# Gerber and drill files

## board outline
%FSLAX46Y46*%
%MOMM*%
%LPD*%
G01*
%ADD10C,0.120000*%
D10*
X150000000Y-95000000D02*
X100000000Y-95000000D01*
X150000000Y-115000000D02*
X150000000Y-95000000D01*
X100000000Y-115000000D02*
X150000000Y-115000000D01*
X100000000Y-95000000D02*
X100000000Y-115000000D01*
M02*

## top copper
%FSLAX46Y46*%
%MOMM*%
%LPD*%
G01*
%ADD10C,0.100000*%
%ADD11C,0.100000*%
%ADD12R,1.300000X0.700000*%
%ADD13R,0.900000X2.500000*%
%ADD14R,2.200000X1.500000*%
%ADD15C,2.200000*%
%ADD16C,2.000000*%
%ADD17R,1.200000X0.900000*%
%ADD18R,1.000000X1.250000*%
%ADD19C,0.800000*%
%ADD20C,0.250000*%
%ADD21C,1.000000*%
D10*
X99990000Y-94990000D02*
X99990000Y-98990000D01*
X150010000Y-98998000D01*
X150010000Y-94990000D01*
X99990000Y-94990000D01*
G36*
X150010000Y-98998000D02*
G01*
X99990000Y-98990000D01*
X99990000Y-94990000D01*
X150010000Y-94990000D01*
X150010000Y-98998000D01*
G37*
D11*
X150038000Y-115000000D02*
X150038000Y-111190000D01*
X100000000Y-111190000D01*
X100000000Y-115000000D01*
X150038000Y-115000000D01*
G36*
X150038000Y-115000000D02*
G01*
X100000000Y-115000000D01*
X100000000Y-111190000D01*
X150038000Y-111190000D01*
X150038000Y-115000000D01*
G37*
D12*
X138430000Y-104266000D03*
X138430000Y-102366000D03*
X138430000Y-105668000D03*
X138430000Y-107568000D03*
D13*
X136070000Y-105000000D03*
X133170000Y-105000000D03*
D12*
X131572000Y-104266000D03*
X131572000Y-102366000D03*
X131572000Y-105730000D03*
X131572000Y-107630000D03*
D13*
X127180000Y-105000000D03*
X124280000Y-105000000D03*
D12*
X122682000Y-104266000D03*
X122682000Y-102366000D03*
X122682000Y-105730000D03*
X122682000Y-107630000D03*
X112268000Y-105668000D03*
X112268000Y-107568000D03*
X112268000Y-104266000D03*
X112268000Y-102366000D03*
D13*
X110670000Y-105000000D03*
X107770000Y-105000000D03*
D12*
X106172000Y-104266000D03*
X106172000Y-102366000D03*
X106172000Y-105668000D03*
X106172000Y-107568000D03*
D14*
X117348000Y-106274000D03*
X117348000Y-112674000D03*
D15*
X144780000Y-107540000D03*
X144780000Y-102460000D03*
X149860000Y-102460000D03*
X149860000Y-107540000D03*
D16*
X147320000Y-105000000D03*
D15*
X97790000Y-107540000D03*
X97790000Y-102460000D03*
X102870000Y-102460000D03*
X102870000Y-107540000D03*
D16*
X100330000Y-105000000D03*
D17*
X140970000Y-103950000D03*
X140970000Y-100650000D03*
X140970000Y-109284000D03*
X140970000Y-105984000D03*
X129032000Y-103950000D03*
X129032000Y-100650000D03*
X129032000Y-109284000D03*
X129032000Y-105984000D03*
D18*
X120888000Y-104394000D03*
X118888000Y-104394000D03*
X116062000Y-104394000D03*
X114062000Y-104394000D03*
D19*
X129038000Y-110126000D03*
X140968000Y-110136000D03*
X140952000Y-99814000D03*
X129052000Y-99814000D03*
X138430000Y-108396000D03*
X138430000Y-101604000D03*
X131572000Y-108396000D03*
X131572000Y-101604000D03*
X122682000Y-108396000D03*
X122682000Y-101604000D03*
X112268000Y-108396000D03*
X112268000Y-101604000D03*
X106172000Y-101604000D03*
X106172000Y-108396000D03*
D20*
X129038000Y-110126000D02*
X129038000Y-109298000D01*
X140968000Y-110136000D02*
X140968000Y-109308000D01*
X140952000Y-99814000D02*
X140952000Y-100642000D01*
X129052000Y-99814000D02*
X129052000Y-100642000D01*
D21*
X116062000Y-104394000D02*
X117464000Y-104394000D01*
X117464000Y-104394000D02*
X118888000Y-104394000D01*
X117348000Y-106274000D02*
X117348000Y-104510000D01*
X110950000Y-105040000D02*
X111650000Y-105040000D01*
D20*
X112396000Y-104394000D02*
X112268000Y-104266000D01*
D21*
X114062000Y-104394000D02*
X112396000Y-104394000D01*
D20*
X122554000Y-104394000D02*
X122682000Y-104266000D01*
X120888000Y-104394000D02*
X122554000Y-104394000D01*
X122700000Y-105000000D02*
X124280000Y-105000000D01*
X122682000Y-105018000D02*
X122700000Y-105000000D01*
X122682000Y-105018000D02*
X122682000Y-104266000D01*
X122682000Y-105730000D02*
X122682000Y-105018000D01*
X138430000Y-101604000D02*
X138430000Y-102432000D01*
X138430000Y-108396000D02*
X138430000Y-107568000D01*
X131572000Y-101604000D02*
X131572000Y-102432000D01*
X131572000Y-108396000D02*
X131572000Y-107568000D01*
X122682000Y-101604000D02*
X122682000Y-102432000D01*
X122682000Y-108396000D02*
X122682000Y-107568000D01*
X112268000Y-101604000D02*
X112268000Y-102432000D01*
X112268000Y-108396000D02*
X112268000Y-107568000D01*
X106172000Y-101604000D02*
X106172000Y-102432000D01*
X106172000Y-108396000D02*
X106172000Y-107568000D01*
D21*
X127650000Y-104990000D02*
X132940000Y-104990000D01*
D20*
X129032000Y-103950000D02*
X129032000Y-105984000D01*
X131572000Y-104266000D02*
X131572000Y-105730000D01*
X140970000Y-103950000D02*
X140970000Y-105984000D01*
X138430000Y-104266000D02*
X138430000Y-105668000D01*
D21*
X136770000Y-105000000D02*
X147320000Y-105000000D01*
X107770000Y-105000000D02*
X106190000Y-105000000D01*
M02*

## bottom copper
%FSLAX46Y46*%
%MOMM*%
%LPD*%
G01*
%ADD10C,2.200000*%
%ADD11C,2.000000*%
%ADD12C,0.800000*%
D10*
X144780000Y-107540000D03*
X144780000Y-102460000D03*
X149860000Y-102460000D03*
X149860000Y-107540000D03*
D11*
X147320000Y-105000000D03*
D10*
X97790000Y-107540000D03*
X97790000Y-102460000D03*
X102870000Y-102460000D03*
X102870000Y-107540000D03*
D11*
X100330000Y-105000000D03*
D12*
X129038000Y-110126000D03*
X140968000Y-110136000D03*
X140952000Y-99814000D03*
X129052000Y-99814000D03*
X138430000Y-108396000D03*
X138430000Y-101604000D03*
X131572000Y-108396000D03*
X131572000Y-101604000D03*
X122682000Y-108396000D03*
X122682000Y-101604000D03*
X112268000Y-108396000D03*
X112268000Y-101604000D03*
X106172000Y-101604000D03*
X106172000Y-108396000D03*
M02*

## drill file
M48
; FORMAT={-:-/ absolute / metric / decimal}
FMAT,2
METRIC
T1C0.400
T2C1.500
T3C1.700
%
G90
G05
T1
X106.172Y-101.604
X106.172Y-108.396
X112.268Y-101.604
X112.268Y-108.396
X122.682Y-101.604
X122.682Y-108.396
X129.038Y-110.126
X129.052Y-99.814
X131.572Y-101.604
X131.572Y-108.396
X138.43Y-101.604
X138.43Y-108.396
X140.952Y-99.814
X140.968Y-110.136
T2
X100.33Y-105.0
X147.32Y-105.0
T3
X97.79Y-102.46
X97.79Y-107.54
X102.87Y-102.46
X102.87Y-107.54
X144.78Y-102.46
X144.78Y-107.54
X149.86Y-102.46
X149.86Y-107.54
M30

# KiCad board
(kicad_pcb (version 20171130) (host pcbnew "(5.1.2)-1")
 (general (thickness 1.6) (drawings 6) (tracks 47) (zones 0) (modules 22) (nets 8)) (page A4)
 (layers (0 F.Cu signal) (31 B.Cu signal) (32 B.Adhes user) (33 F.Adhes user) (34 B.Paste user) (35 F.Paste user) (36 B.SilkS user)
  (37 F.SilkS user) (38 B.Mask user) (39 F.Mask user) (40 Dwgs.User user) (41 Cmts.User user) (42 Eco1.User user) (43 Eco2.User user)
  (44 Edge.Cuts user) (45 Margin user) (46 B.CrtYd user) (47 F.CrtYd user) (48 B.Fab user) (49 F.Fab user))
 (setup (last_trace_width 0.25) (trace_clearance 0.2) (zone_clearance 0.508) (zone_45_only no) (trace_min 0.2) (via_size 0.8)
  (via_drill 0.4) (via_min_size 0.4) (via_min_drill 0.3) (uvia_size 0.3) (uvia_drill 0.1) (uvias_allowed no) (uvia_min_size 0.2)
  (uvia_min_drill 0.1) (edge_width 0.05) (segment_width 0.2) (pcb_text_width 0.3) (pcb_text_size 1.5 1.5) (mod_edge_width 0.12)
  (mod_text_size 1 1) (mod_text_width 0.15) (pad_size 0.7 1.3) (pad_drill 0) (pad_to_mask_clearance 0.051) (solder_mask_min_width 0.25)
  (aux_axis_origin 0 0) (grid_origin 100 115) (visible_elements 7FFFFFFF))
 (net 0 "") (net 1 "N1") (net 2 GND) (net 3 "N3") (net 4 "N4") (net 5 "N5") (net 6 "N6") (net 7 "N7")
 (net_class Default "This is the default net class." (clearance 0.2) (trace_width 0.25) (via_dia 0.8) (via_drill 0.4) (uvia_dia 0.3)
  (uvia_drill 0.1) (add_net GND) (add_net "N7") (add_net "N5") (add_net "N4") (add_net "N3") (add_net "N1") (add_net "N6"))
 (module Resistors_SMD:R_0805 (layer F.Cu) (at 138.43 103.316 90)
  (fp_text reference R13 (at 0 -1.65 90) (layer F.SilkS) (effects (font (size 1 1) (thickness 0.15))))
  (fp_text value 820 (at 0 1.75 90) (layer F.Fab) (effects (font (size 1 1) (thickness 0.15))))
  (pad 1 smd rect (at -0.95 0 90) (size 0.7 1.3) (layers F.Cu F.Paste F.Mask) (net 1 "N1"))
  (pad 2 smd rect (at 0.95 0 90) (size 0.7 1.3) (layers F.Cu F.Paste F.Mask) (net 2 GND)))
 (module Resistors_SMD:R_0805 (layer F.Cu) (at 138.43 106.618 270)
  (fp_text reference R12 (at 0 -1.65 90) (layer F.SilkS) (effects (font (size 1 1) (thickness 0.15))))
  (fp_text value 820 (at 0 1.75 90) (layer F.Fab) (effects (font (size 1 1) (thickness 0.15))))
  (pad 1 smd rect (at -0.95 0 270) (size 0.7 1.3) (layers F.Cu F.Paste F.Mask) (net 1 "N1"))
  (pad 2 smd rect (at 0.95 0 270) (size 0.7 1.3) (layers F.Cu F.Paste F.Mask) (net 2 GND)))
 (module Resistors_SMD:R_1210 (layer F.Cu) (at 134.62 105 180)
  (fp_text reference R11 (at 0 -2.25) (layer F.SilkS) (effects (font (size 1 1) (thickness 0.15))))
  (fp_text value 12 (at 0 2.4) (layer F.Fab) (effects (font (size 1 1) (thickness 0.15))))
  (pad 1 smd rect (at -1.45 0 180) (size 0.9 2.5) (layers F.Cu F.Paste F.Mask) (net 1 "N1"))
  (pad 2 smd rect (at 1.45 0 180) (size 0.9 2.5) (layers F.Cu F.Paste F.Mask) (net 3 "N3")))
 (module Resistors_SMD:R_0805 (layer F.Cu) (at 131.572 103.316 90)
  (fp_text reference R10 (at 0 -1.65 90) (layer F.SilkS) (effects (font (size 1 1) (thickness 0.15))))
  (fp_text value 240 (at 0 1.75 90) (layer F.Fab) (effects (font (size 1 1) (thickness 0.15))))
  (pad 1 smd rect (at -0.95 0 90) (size 0.7 1.3) (layers F.Cu F.Paste F.Mask) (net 3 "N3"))
  (pad 2 smd rect (at 0.95 0 90) (size 0.7 1.3) (layers F.Cu F.Paste F.Mask) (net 2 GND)))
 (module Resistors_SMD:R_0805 (layer F.Cu) (at 131.572 106.68 270)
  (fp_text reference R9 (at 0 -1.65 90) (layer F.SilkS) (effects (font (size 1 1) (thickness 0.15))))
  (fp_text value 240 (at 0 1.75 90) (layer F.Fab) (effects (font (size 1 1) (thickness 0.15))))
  (pad 1 smd rect (at -0.95 0 270) (size 0.7 1.3) (layers F.Cu F.Paste F.Mask) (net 3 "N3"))
  (pad 2 smd rect (at 0.95 0 270) (size 0.7 1.3) (layers F.Cu F.Paste F.Mask) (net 2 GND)))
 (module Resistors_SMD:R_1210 (layer F.Cu) (at 125.73 105 180)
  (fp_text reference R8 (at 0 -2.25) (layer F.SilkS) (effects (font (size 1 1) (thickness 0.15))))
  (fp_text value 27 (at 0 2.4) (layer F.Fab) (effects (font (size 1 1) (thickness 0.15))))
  (pad 1 smd rect (at -1.45 0 180) (size 0.9 2.5) (layers F.Cu F.Paste F.Mask) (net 3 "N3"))
  (pad 2 smd rect (at 1.45 0 180) (size 0.9 2.5) (layers F.Cu F.Paste F.Mask) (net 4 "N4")))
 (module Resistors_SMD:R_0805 (layer F.Cu) (at 122.682 103.316 90)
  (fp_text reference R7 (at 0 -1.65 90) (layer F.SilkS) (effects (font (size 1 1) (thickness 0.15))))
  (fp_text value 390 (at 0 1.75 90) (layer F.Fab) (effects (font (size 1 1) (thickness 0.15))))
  (pad 1 smd rect (at -0.95 0 90) (size 0.7 1.3) (layers F.Cu F.Paste F.Mask) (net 4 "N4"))
  (pad 2 smd rect (at 0.95 0 90) (size 0.7 1.3) (layers F.Cu F.Paste F.Mask) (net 2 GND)))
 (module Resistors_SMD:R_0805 (layer F.Cu) (at 122.682 106.68 270)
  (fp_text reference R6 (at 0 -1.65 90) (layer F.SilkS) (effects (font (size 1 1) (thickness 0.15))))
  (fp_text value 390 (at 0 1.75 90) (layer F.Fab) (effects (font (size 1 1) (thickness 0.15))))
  (pad 1 smd rect (at -0.95 0 270) (size 0.7 1.3) (layers F.Cu F.Paste F.Mask) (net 4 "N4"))
  (pad 2 smd rect (at 0.95 0 270) (size 0.7 1.3) (layers F.Cu F.Paste F.Mask) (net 2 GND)))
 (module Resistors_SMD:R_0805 (layer F.Cu) (at 112.268 106.618 270)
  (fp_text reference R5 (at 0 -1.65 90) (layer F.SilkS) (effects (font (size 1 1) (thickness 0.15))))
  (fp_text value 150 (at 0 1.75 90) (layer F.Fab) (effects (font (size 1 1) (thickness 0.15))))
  (pad 1 smd rect (at -0.95 0 270) (size 0.7 1.3) (layers F.Cu F.Paste F.Mask) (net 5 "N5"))
  (pad 2 smd rect (at 0.95 0 270) (size 0.7 1.3) (layers F.Cu F.Paste F.Mask) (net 2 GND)))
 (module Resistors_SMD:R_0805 (layer F.Cu) (at 112.268 103.316 90)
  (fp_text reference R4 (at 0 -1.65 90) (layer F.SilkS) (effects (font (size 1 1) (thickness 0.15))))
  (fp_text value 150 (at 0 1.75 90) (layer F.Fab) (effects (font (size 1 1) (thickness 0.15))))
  (pad 1 smd rect (at -0.95 0 90) (size 0.7 1.3) (layers F.Cu F.Paste F.Mask) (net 5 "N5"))
  (pad 2 smd rect (at 0.95 0 90) (size 0.7 1.3) (layers F.Cu F.Paste F.Mask) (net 2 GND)))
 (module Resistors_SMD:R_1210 (layer F.Cu) (at 109.22 105 180)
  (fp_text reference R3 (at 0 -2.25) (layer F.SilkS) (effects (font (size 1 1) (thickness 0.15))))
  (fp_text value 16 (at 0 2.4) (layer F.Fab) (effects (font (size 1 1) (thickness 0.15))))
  (pad 1 smd rect (at -1.45 0 180) (size 0.9 2.5) (layers F.Cu F.Paste F.Mask) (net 5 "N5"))
  (pad 2 smd rect (at 1.45 0 180) (size 0.9 2.5) (layers F.Cu F.Paste F.Mask) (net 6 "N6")))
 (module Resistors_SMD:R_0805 (layer F.Cu) (at 106.172 103.316 90)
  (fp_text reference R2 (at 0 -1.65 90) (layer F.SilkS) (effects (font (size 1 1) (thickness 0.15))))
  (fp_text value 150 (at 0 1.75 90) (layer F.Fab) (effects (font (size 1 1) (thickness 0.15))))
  (pad 1 smd rect (at -0.95 0 90) (size 0.7 1.3) (layers F.Cu F.Paste F.Mask) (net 6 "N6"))
  (pad 2 smd rect (at 0.95 0 90) (size 0.7 1.3) (layers F.Cu F.Paste F.Mask) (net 2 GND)))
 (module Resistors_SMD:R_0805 (layer F.Cu) (at 106.172 106.618 270)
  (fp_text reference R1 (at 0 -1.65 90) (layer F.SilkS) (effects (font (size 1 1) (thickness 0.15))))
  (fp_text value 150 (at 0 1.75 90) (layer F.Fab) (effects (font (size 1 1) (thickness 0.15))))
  (pad 1 smd rect (at -0.95 0 270) (size 0.7 1.3) (layers F.Cu F.Paste F.Mask) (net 6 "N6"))
  (pad 2 smd rect (at 0.95 0 270) (size 0.7 1.3) (layers F.Cu F.Paste F.Mask) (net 2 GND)))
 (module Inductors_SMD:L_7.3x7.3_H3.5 (layer F.Cu) (at 117.348 109.474 270)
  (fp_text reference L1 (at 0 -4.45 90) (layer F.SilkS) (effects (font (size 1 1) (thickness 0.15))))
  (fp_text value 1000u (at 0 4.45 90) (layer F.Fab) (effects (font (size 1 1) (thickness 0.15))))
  (pad 1 smd rect (at -3.2 0 270) (size 1.5 2.2) (layers F.Cu F.Paste F.Mask) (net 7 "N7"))
  (pad 2 smd rect (at 3.2 0 270) (size 1.5 2.2) (layers F.Cu F.Paste F.Mask) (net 2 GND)))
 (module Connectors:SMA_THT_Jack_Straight (layer F.Cu) (at 147.32 105)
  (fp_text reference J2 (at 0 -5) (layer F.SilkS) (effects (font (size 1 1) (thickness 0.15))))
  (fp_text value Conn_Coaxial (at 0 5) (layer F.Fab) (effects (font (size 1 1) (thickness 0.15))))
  (pad 2 thru_hole circle (at -2.54 2.54) (size 2.2 2.2) (drill 1.7) (layers *.Cu *.Mask) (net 2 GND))
  (pad 2 thru_hole circle (at -2.54 -2.54) (size 2.2 2.2) (drill 1.7) (layers *.Cu *.Mask) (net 2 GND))
  (pad 2 thru_hole circle (at 2.54 -2.54) (size 2.2 2.2) (drill 1.7) (layers *.Cu *.Mask) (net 2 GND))
  (pad 2 thru_hole circle (at 2.54 2.54) (size 2.2 2.2) (drill 1.7) (layers *.Cu *.Mask) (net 2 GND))
  (pad 1 thru_hole circle (at 0 0) (size 2 2) (drill 1.5) (layers *.Cu *.Mask) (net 1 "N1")))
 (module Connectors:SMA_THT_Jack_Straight (layer F.Cu) (at 100.33 105)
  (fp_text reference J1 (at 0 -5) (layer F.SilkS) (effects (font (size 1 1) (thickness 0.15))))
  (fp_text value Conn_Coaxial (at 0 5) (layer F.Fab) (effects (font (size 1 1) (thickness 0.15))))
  (pad 2 thru_hole circle (at -2.54 2.54) (size 2.2 2.2) (drill 1.7) (layers *.Cu *.Mask) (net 2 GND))
  (pad 2 thru_hole circle (at -2.54 -2.54) (size 2.2 2.2) (drill 1.7) (layers *.Cu *.Mask) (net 2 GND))
  (pad 2 thru_hole circle (at 2.54 -2.54) (size 2.2 2.2) (drill 1.7) (layers *.Cu *.Mask) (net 2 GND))
  (pad 2 thru_hole circle (at 2.54 2.54) (size 2.2 2.2) (drill 1.7) (layers *.Cu *.Mask) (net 2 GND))
  (pad 1 thru_hole circle (at 0 0) (size 2 2) (drill 1.5) (layers *.Cu *.Mask) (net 6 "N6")))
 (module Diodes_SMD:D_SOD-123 (layer F.Cu) (at 140.97 102.3 90)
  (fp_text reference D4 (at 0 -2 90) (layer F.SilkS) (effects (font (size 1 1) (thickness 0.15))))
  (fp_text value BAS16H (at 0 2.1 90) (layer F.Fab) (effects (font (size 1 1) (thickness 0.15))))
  (pad 1 smd rect (at -1.65 0 90) (size 0.9 1.2) (layers F.Cu F.Paste F.Mask) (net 1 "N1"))
  (pad 2 smd rect (at 1.65 0 90) (size 0.9 1.2) (layers F.Cu F.Paste F.Mask) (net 2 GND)))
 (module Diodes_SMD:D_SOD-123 (layer F.Cu) (at 140.97 107.634 90)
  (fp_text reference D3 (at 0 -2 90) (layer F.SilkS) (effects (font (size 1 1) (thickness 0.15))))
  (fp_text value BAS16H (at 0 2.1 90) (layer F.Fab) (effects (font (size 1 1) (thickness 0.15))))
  (pad 1 smd rect (at -1.65 0 90) (size 0.9 1.2) (layers F.Cu F.Paste F.Mask) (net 2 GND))
  (pad 2 smd rect (at 1.65 0 90) (size 0.9 1.2) (layers F.Cu F.Paste F.Mask) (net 1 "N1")))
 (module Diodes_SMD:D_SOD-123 (layer F.Cu) (at 129.032 102.3 90)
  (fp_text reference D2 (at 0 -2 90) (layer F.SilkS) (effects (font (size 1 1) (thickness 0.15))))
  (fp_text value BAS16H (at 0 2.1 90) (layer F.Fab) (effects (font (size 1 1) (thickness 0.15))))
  (pad 1 smd rect (at -1.65 0 90) (size 0.9 1.2) (layers F.Cu F.Paste F.Mask) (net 3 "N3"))
  (pad 2 smd rect (at 1.65 0 90) (size 0.9 1.2) (layers F.Cu F.Paste F.Mask) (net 2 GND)))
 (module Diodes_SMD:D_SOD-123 (layer F.Cu) (at 129.032 107.634 90)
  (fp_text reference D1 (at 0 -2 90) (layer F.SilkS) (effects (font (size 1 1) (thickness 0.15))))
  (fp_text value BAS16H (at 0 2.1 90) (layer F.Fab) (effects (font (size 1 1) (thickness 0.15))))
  (pad 1 smd rect (at -1.65 0 90) (size 0.9 1.2) (layers F.Cu F.Paste F.Mask) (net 2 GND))
  (pad 2 smd rect (at 1.65 0 90) (size 0.9 1.2) (layers F.Cu F.Paste F.Mask) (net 3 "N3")))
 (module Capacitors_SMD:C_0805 (layer F.Cu) (at 119.888 104.394 180)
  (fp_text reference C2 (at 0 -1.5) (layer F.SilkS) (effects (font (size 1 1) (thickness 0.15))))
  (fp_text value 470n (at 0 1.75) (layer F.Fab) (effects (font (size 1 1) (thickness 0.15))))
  (pad 1 smd rect (at -1 0 180) (size 1 1.25) (layers F.Cu F.Paste F.Mask) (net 4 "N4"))
  (pad 2 smd rect (at 1 0 180) (size 1 1.25) (layers F.Cu F.Paste F.Mask) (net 7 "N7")))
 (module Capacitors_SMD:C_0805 (layer F.Cu) (at 115.062 104.394 180)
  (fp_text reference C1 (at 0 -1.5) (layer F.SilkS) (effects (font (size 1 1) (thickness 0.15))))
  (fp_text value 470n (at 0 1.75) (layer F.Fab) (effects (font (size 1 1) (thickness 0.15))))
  (pad 1 smd rect (at -1 0 180) (size 1 1.25) (layers F.Cu F.Paste F.Mask) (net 7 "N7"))
  (pad 2 smd rect (at 1 0 180) (size 1 1.25) (layers F.Cu F.Paste F.Mask) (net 5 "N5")))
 (gr_poly (pts (xy 99.99 94.99) (xy 99.99 98.99) (xy 150.01 98.998) (xy 150.01 94.99)) (layer F.Cu) (width 0.1))
 (gr_poly (pts (xy 150.038 115) (xy 150.038 111.19) (xy 100 111.19) (xy 100 115)) (layer F.Cu) (width 0.1))
 (gr_line (start 150 95) (end 100 95) (layer Edge.Cuts) (width 0.12))
 (gr_line (start 150 115) (end 150 95) (layer Edge.Cuts) (width 0.12))
 (gr_line (start 100 115) (end 150 115) (layer Edge.Cuts) (width 0.12))
 (gr_line (start 100 95) (end 100 115) (layer Edge.Cuts) (width 0.12))
 (via (at 129.038 110.126) (size 0.8) (drill 0.4) (layers F.Cu B.Cu) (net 2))
 (segment (start 129.038 110.126) (end 129.038 109.298) (width 0.25) (layer F.Cu) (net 2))
 (via (at 140.968 110.136) (size 0.8) (drill 0.4) (layers F.Cu B.Cu) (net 2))
 (segment (start 140.968 110.136) (end 140.968 109.308) (width 0.25) (layer F.Cu) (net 2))
 (via (at 140.952 99.814) (size 0.8) (drill 0.4) (layers F.Cu B.Cu) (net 2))
 (segment (start 140.952 99.814) (end 140.952 100.642) (width 0.25) (layer F.Cu) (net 2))
 (via (at 129.052 99.814) (size 0.8) (drill 0.4) (layers F.Cu B.Cu) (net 2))
 (segment (start 129.052 99.814) (end 129.052 100.642) (width 0.25) (layer F.Cu) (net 2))
 (segment (start 116.062 104.394) (end 117.464 104.394) (width 1) (layer F.Cu) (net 7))
 (segment (start 117.464 104.394) (end 118.888 104.394) (width 1) (layer F.Cu) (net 7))
 (segment (start 117.348 106.274) (end 117.348 104.51) (width 1) (layer F.Cu) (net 7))
 (segment (start 110.95 105.04) (end 111.65 105.04) (width 1) (layer F.Cu) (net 5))
 (segment (start 112.396 104.394) (end 112.268 104.266) (width 0.25) (layer F.Cu) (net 5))
 (segment (start 114.062 104.394) (end 112.396 104.394) (width 1) (layer F.Cu) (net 5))
 (segment (start 122.554 104.394) (end 122.682 104.266) (width 0.25) (layer F.Cu) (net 4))
 (segment (start 120.888 104.394) (end 122.554 104.394) (width 0.25) (layer F.Cu) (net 4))
 (segment (start 122.7 105) (end 124.28 105) (width 0.25) (layer F.Cu) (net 4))
 (segment (start 122.682 105.018) (end 122.7 105) (width 0.25) (layer F.Cu) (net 4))
 (segment (start 122.682 105.018) (end 122.682 104.266) (width 0.25) (layer F.Cu) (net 4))
 (segment (start 122.682 105.73) (end 122.682 105.018) (width 0.25) (layer F.Cu) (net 4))
 (segment (start 138.43 101.604) (end 138.43 102.432) (width 0.25) (layer F.Cu) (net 2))
 (segment (start 138.43 108.396) (end 138.43 107.568) (width 0.25) (layer F.Cu) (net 2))
 (via (at 138.43 108.396) (size 0.8) (drill 0.4) (layers F.Cu B.Cu) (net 2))
 (via (at 138.43 101.604) (size 0.8) (drill 0.4) (layers F.Cu B.Cu) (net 2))
 (segment (start 131.572 101.604) (end 131.572 102.432) (width 0.25) (layer F.Cu) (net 2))
 (segment (start 131.572 108.396) (end 131.572 107.568) (width 0.25) (layer F.Cu) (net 2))
 (via (at 131.572 108.396) (size 0.8) (drill 0.4) (layers F.Cu B.Cu) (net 2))
 (via (at 131.572 101.604) (size 0.8) (drill 0.4) (layers F.Cu B.Cu) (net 2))
 (segment (start 122.682 101.604) (end 122.682 102.432) (width 0.25) (layer F.Cu) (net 2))
 (segment (start 122.682 108.396) (end 122.682 107.568) (width 0.25) (layer F.Cu) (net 2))
 (via (at 122.682 108.396) (size 0.8) (drill 0.4) (layers F.Cu B.Cu) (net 2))
 (via (at 122.682 101.604) (size 0.8) (drill 0.4) (layers F.Cu B.Cu) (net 2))
 (segment (start 112.268 101.604) (end 112.268 102.432) (width 0.25) (layer F.Cu) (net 2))
 (segment (start 112.268 108.396) (end 112.268 107.568) (width 0.25) (layer F.Cu) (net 2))
 (via (at 112.268 108.396) (size 0.8) (drill 0.4) (layers F.Cu B.Cu) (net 2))
 (via (at 112.268 101.604) (size 0.8) (drill 0.4) (layers F.Cu B.Cu) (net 2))
 (segment (start 106.172 101.604) (end 106.172 102.432) (width 0.25) (layer F.Cu) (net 2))
 (via (at 106.172 101.604) (size 0.8) (drill 0.4) (layers F.Cu B.Cu) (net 2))
 (via (at 106.172 108.396) (size 0.8) (drill 0.4) (layers F.Cu B.Cu) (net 2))
 (segment (start 106.172 108.396) (end 106.172 107.568) (width 0.25) (layer F.Cu) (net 2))
 (segment (start 127.65 104.99) (end 132.94 104.99) (width 1) (layer F.Cu) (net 3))
 (segment (start 129.032 103.95) (end 129.032 105.984) (width 0.25) (layer F.Cu) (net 3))
 (segment (start 131.572 104.266) (end 131.572 105.73) (width 0.25) (layer F.Cu) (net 3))
 (segment (start 140.97 103.95) (end 140.97 105.984) (width 0.25) (layer F.Cu) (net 1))
 (segment (start 138.43 104.266) (end 138.43 105.668) (width 0.25) (layer F.Cu) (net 1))
 (segment (start 136.77 105) (end 147.32 105) (width 1) (layer F.Cu) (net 1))
 (segment (start 107.77 105) (end 106.19 105) (width 1) (layer F.Cu) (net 6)))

